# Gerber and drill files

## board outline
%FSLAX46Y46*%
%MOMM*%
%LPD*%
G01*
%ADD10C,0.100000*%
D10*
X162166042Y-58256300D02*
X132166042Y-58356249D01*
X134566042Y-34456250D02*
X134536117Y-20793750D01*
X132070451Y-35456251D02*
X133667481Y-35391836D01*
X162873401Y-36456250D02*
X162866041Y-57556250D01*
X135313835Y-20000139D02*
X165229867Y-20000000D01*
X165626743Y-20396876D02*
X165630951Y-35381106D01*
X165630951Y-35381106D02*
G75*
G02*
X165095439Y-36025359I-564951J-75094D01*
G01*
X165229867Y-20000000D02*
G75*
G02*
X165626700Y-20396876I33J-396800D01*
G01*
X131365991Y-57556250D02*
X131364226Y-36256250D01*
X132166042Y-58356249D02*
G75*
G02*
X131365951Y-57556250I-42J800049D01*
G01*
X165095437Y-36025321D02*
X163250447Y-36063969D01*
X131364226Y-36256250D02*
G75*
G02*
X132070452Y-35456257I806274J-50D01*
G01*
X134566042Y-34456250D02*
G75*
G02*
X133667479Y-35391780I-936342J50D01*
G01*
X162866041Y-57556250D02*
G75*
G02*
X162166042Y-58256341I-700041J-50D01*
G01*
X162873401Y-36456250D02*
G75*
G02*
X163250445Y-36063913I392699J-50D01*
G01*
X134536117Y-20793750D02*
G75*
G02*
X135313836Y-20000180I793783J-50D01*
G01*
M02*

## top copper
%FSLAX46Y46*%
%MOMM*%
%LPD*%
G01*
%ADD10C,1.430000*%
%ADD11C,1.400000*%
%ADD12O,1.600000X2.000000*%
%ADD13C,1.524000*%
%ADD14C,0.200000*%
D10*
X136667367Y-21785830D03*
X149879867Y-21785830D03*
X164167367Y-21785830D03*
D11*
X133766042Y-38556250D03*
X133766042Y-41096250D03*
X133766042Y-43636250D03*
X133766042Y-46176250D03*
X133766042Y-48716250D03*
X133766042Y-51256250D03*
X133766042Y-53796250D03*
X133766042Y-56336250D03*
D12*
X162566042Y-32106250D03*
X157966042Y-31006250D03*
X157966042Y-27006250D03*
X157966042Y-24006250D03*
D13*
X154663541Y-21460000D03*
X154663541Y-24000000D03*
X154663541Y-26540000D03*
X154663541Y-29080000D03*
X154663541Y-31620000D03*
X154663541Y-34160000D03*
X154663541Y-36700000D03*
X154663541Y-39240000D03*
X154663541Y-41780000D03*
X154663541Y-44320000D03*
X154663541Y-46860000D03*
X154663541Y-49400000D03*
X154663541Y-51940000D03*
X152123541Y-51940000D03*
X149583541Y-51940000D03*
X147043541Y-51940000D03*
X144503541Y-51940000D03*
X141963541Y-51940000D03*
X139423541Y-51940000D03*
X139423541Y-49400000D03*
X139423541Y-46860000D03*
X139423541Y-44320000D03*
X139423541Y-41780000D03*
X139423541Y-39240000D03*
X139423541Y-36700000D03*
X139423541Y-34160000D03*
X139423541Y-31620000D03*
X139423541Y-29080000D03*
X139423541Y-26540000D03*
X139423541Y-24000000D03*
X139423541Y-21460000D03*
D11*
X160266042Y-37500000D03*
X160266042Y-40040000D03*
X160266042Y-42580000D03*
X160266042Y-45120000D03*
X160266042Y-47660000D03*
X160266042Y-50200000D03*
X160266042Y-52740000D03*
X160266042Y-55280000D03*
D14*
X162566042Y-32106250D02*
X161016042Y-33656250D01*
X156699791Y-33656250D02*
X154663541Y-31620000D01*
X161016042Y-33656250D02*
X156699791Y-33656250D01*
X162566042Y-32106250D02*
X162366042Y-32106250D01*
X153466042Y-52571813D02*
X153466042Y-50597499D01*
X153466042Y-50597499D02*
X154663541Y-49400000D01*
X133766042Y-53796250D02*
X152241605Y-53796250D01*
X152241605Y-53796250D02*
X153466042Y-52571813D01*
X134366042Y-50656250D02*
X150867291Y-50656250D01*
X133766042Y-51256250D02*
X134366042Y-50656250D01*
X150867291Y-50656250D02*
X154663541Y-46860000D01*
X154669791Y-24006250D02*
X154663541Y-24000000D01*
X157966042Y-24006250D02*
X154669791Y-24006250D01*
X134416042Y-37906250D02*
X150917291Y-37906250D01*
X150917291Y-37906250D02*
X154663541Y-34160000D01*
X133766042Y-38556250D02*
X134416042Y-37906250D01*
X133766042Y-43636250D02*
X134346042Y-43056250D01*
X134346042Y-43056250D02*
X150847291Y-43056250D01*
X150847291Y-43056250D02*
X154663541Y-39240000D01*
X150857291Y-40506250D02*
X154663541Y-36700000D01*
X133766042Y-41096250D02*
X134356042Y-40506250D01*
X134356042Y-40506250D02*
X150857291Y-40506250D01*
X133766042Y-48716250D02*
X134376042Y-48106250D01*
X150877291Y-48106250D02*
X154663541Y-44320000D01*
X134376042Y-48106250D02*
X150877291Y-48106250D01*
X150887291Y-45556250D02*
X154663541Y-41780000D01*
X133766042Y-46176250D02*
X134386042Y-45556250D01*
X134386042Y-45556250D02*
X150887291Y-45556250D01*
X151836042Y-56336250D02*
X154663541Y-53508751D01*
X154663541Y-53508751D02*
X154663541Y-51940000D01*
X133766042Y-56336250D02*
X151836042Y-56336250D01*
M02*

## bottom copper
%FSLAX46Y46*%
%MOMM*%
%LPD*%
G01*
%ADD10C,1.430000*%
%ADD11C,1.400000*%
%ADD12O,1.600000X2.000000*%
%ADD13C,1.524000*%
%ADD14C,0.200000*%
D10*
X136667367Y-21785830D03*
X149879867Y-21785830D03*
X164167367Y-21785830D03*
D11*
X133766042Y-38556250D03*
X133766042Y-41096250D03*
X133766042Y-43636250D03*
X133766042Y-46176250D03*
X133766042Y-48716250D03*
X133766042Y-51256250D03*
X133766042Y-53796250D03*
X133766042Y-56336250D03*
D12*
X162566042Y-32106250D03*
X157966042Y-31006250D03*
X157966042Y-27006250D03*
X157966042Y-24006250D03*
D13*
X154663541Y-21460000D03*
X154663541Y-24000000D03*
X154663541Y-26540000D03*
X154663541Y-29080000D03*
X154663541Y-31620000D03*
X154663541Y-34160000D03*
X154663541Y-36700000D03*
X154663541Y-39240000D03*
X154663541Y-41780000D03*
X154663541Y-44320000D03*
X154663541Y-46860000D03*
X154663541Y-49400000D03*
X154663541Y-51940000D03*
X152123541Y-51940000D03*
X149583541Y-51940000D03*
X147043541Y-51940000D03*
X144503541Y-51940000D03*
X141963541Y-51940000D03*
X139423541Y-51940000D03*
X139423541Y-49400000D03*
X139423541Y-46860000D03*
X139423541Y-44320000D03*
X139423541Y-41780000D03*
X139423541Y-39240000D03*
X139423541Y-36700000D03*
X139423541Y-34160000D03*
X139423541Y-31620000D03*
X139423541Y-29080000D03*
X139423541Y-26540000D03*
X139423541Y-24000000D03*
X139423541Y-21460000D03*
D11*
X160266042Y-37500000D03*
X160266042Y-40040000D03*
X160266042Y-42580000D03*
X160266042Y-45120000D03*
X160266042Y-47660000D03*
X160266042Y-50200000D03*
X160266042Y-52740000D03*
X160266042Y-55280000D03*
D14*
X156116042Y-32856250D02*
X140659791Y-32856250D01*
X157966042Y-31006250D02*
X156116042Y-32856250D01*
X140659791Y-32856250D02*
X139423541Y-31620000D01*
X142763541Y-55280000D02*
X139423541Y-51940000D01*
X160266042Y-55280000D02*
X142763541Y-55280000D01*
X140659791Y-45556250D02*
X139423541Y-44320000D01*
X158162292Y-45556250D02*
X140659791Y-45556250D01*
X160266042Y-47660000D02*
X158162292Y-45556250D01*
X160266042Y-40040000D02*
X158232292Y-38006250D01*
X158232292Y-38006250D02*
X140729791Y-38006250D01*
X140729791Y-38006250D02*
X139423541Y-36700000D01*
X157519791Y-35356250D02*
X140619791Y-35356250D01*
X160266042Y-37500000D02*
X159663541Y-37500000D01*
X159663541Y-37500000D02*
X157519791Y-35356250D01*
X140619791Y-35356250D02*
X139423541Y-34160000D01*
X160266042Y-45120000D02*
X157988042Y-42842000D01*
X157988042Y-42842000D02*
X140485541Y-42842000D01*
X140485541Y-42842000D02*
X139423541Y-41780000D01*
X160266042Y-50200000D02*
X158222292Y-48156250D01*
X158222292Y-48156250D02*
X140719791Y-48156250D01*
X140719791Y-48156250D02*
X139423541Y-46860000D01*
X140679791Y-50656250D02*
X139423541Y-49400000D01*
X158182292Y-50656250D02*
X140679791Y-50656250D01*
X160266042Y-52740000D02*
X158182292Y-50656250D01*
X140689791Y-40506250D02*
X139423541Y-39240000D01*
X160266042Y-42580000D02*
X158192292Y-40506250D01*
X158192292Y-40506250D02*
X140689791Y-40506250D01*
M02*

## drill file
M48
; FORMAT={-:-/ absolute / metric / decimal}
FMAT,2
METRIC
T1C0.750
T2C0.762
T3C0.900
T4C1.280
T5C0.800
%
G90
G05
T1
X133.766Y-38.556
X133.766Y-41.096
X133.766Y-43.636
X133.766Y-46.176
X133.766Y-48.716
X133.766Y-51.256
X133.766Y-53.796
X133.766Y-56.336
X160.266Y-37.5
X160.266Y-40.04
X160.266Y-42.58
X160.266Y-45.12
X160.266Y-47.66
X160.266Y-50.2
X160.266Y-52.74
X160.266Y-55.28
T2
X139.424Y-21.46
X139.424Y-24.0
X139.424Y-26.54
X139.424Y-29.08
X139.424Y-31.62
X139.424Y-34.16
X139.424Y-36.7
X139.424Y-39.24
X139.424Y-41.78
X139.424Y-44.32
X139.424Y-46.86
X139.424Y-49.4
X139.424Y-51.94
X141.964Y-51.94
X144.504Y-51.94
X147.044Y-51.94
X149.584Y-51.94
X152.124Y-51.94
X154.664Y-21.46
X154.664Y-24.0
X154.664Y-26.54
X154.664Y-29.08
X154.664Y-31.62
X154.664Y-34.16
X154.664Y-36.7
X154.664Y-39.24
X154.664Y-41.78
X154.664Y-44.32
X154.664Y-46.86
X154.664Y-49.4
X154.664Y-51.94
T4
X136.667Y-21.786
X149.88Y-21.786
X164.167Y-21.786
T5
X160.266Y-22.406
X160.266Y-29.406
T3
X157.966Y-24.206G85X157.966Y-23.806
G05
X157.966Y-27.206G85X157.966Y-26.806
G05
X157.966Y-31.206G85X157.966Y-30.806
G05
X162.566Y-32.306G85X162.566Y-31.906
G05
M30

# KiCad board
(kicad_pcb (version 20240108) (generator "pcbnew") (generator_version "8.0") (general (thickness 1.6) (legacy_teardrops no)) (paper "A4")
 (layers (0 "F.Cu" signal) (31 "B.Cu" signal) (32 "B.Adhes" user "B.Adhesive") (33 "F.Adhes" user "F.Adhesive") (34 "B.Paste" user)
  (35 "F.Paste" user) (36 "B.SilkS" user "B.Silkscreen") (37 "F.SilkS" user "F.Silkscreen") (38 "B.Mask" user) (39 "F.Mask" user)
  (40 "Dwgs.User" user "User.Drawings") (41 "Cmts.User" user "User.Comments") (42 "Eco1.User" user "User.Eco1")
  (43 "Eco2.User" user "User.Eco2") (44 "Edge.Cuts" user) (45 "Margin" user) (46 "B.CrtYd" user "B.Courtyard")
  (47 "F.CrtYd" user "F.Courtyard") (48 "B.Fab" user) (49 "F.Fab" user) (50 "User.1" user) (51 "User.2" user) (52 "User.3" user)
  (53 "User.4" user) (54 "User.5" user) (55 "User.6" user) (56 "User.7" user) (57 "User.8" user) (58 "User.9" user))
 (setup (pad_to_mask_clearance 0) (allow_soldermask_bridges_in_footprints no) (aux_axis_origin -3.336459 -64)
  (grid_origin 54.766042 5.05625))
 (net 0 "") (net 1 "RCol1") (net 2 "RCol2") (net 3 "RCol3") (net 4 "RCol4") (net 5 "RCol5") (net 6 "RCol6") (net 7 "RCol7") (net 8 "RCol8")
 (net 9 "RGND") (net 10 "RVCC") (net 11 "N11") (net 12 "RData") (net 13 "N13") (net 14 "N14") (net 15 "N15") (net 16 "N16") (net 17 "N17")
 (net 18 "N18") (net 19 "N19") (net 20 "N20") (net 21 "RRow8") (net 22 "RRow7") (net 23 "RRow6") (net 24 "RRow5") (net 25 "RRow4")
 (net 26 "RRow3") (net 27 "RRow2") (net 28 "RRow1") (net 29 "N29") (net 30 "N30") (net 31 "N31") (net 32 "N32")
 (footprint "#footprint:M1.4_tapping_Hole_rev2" (layer "F.Cu") (at 146.916042 21.90625 -90)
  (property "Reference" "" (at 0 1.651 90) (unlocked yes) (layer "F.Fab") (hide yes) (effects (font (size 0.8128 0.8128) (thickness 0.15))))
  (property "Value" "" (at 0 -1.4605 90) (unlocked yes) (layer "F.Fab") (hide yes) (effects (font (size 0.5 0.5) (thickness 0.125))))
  (pad "" thru_hole circle (at -0.12042 10.248675 270) (size 1.43 1.43) (drill 1.28) (layers "*.Cu" "*.Mask") (remove_unused_layers no)))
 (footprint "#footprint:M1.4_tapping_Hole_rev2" (layer "F.Cu") (at 149.879867 21.78583 -90)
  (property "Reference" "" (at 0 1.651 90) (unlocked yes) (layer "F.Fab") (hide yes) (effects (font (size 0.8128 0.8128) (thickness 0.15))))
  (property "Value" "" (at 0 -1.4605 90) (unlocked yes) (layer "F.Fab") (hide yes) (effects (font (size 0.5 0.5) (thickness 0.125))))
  (pad "" thru_hole circle (at 0 0 270) (size 1.43 1.43) (drill 1.28) (layers "*.Cu" "*.Mask") (remove_unused_layers no)))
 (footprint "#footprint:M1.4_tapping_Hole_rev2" (layer "F.Cu") (at 164.167367 21.78583 -90)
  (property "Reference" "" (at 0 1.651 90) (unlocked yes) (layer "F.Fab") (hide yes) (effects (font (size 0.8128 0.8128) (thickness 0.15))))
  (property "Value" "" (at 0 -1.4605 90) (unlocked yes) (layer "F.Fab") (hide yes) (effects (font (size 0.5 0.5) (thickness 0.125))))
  (pad "" thru_hole circle (at 0 0 270) (size 1.43 1.43) (drill 1.28) (layers "*.Cu" "*.Mask") (remove_unused_layers no)))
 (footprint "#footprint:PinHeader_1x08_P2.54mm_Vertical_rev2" (layer "B.Cu") (at 133.766042 38.55625 180)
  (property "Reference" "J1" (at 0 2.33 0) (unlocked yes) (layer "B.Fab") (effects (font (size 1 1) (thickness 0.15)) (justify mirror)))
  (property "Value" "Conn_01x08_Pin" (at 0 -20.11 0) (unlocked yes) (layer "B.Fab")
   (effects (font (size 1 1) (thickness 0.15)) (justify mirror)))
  (pad "1" thru_hole circle (at 0 0 180) (size 1.4 1.4) (drill 0.75) (layers "*.Cu" "*.Mask") (remove_unused_layers no) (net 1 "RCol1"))
  (pad "2" thru_hole circle (at 0 -2.54 180) (size 1.4 1.4) (drill 0.75) (layers "*.Cu" "*.Mask") (remove_unused_layers no) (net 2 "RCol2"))
  (pad "3" thru_hole circle (at 0 -5.08 180) (size 1.4 1.4) (drill 0.75) (layers "*.Cu" "*.Mask") (remove_unused_layers no) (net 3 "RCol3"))
  (pad "4" thru_hole circle (at 0 -7.62 180) (size 1.4 1.4) (drill 0.75) (layers "*.Cu" "*.Mask") (remove_unused_layers no) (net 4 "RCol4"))
  (pad "5" thru_hole circle (at 0 -10.16 180) (size 1.4 1.4) (drill 0.75) (layers "*.Cu" "*.Mask") (remove_unused_layers no) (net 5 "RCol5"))
  (pad "6" thru_hole circle (at 0 -12.7 180) (size 1.4 1.4) (drill 0.75) (layers "*.Cu" "*.Mask") (remove_unused_layers no) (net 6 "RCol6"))
  (pad "7" thru_hole circle (at 0 -15.24 180) (size 1.4 1.4) (drill 0.75) (layers "*.Cu" "*.Mask") (remove_unused_layers no) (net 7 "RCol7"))
  (pad "8" thru_hole circle (at 0 -17.78 180) (size 1.4 1.4) (drill 0.75) (layers "*.Cu" "*.Mask") (remove_unused_layers no) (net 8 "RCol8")))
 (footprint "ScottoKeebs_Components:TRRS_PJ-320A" (layer "B.Cu") (at 160.266042 20.80625 180)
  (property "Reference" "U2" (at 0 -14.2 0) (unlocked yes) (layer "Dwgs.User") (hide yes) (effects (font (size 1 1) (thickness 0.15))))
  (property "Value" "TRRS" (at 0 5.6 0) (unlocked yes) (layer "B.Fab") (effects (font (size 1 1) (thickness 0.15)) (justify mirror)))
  (pad "" np_thru_hole circle (at 0 -8.6 180) (size 0.8 0.8) (drill 0.8) (layers "*.Cu" "*.Mask"))
  (pad "" np_thru_hole circle (at 0 -1.6 180) (size 0.8 0.8) (drill 0.8) (layers "*.Cu" "*.Mask"))
  (pad "1" thru_hole oval (at -2.3 -11.3 180) (size 1.6 2) (drill oval 0.9 1.3) (layers "*.Cu" "*.Mask") (remove_unused_layers no)
   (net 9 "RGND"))
  (pad "2" thru_hole oval (at 2.3 -10.2 180) (size 1.6 2) (drill oval 0.9 1.3) (layers "*.Cu" "*.Mask") (remove_unused_layers no)
   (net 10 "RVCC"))
  (pad "3" thru_hole oval (at 2.3 -6.2 180) (size 1.6 2) (drill oval 0.9 1.3) (layers "*.Cu" "*.Mask") (remove_unused_layers no)
   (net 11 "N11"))
  (pad "4" thru_hole oval (at 2.3 -3.2 180) (size 1.6 2) (drill oval 0.9 1.3) (layers "*.Cu" "*.Mask") (remove_unused_layers no)
   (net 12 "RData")))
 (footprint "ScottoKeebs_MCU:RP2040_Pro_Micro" (layer "B.Cu") (at 147.043541 37.97 180)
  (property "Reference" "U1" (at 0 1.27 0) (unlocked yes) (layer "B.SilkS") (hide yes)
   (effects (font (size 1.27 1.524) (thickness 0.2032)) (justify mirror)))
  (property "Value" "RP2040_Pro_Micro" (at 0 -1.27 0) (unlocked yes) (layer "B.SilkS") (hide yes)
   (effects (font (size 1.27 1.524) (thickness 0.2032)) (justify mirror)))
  (pad "1" thru_hole circle (at -7.62 16.51 180) (size 1.524 1.524) (drill 0.762) (layers "*.Cu" "*.Mask") (remove_unused_layers no)
   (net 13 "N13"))
  (pad "2" thru_hole circle (at -7.62 13.97 180) (size 1.524 1.524) (drill 0.762) (layers "*.Cu" "*.Mask") (remove_unused_layers no)
   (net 12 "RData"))
  (pad "3" thru_hole circle (at -7.62 11.43 180) (size 1.524 1.524) (drill 0.762) (layers "*.Cu" "*.Mask") (remove_unused_layers no)
   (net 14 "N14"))
  (pad "4" thru_hole circle (at -7.62 8.89 180) (size 1.524 1.524) (drill 0.762) (layers "*.Cu" "*.Mask") (remove_unused_layers no)
   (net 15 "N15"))
  (pad "5" thru_hole circle (at -7.62 6.35 180) (size 1.524 1.524) (drill 0.762) (layers "*.Cu" "*.Mask") (remove_unused_layers no)
   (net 9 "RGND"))
  (pad "6" thru_hole circle (at -7.62 3.81 180) (size 1.524 1.524) (drill 0.762) (layers "*.Cu" "*.Mask") (remove_unused_layers no)
   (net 1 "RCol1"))
  (pad "7" thru_hole circle (at -7.62 1.27 180) (size 1.524 1.524) (drill 0.762) (layers "*.Cu" "*.Mask") (remove_unused_layers no)
   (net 2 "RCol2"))
  (pad "8" thru_hole circle (at -7.62 -1.27 180) (size 1.524 1.524) (drill 0.762) (layers "*.Cu" "*.Mask") (remove_unused_layers no)
   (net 3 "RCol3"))
  (pad "9" thru_hole circle (at -7.62 -3.81 180) (size 1.524 1.524) (drill 0.762) (layers "*.Cu" "*.Mask") (remove_unused_layers no)
   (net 4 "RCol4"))
  (pad "10" thru_hole circle (at -7.62 -6.35 180) (size 1.524 1.524) (drill 0.762) (layers "*.Cu" "*.Mask") (remove_unused_layers no)
   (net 5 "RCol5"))
  (pad "11" thru_hole circle (at -7.62 -8.89 180) (size 1.524 1.524) (drill 0.762) (layers "*.Cu" "*.Mask") (remove_unused_layers no)
   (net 6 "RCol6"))
  (pad "12" thru_hole circle (at -7.62 -11.43 180) (size 1.524 1.524) (drill 0.762) (layers "*.Cu" "*.Mask") (remove_unused_layers no)
   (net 7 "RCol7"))
  (pad "13" thru_hole circle (at -7.62 -13.97 180) (size 1.524 1.524) (drill 0.762) (layers "*.Cu" "*.Mask") (remove_unused_layers no)
   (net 8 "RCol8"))
  (pad "14" thru_hole circle (at -5.08 -13.97 180) (size 1.524 1.524) (drill 0.762) (layers "*.Cu" "*.Mask") (remove_unused_layers no)
   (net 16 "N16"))
  (pad "15" thru_hole circle (at -2.54 -13.97 180) (size 1.524 1.524) (drill 0.762) (layers "*.Cu" "*.Mask") (remove_unused_layers no)
   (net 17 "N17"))
  (pad "16" thru_hole circle (at 0 -13.97 180) (size 1.524 1.524) (drill 0.762) (layers "*.Cu" "*.Mask") (remove_unused_layers no)
   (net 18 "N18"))
  (pad "17" thru_hole circle (at 2.54 -13.97 180) (size 1.524 1.524) (drill 0.762) (layers "*.Cu" "*.Mask") (remove_unused_layers no)
   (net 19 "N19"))
  (pad "18" thru_hole circle (at 5.08 -13.97 180) (size 1.524 1.524) (drill 0.762) (layers "*.Cu" "*.Mask") (remove_unused_layers no)
   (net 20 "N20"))
  (pad "19" thru_hole circle (at 7.62 -13.97 180) (size 1.524 1.524) (drill 0.762) (layers "*.Cu" "*.Mask") (remove_unused_layers no)
   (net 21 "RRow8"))
  (pad "20" thru_hole circle (at 7.62 -11.43 180) (size 1.524 1.524) (drill 0.762) (layers "*.Cu" "*.Mask") (remove_unused_layers no)
   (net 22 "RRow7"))
  (pad "21" thru_hole circle (at 7.62 -8.89 180) (size 1.524 1.524) (drill 0.762) (layers "*.Cu" "*.Mask") (remove_unused_layers no)
   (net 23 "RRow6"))
  (pad "22" thru_hole circle (at 7.62 -6.35 180) (size 1.524 1.524) (drill 0.762) (layers "*.Cu" "*.Mask") (remove_unused_layers no)
   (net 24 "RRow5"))
  (pad "23" thru_hole circle (at 7.62 -3.81 180) (size 1.524 1.524) (drill 0.762) (layers "*.Cu" "*.Mask") (remove_unused_layers no)
   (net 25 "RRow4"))
  (pad "24" thru_hole circle (at 7.62 -1.27 180) (size 1.524 1.524) (drill 0.762) (layers "*.Cu" "*.Mask") (remove_unused_layers no)
   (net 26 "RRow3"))
  (pad "25" thru_hole circle (at 7.62 1.27 180) (size 1.524 1.524) (drill 0.762) (layers "*.Cu" "*.Mask") (remove_unused_layers no)
   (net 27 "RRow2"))
  (pad "26" thru_hole circle (at 7.62 3.81 180) (size 1.524 1.524) (drill 0.762) (layers "*.Cu" "*.Mask") (remove_unused_layers no)
   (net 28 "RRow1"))
  (pad "27" thru_hole circle (at 7.62 6.35 180) (size 1.524 1.524) (drill 0.762) (layers "*.Cu" "*.Mask") (remove_unused_layers no)
   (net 10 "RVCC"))
  (pad "28" thru_hole circle (at 7.62 8.89 180) (size 1.524 1.524) (drill 0.762) (layers "*.Cu" "*.Mask") (remove_unused_layers no)
   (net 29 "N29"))
  (pad "29" thru_hole circle (at 7.62 11.43 180) (size 1.524 1.524) (drill 0.762) (layers "*.Cu" "*.Mask") (remove_unused_layers no)
   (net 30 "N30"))
  (pad "30" thru_hole circle (at 7.62 13.97 180) (size 1.524 1.524) (drill 0.762) (layers "*.Cu" "*.Mask") (remove_unused_layers no)
   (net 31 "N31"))
  (pad "31" thru_hole circle (at 7.62 16.51 180) (size 1.524 1.524) (drill 0.762) (layers "*.Cu" "*.Mask") (remove_unused_layers no)
   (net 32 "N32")))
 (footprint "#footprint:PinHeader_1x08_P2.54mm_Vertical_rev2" (layer "B.Cu") (at 160.266042 37.5 180)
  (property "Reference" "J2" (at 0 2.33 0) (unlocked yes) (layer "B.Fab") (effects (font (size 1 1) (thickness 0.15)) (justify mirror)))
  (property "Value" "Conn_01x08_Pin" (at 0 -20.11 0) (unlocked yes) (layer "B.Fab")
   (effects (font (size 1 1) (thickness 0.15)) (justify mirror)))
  (pad "1" thru_hole circle (at 0 0 180) (size 1.4 1.4) (drill 0.75) (layers "*.Cu" "*.Mask") (remove_unused_layers no) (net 28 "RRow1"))
  (pad "2" thru_hole circle (at 0 -2.54 180) (size 1.4 1.4) (drill 0.75) (layers "*.Cu" "*.Mask") (remove_unused_layers no) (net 27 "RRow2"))
  (pad "3" thru_hole circle (at 0 -5.08 180) (size 1.4 1.4) (drill 0.75) (layers "*.Cu" "*.Mask") (remove_unused_layers no) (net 26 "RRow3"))
  (pad "4" thru_hole circle (at 0 -7.62 180) (size 1.4 1.4) (drill 0.75) (layers "*.Cu" "*.Mask") (remove_unused_layers no) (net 25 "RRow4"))
  (pad "5" thru_hole circle (at 0 -10.16 180) (size 1.4 1.4) (drill 0.75) (layers "*.Cu" "*.Mask") (remove_unused_layers no)
   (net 24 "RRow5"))
  (pad "6" thru_hole circle (at 0 -12.7 180) (size 1.4 1.4) (drill 0.75) (layers "*.Cu" "*.Mask") (remove_unused_layers no) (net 23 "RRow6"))
  (pad "7" thru_hole circle (at 0 -15.24 180) (size 1.4 1.4) (drill 0.75) (layers "*.Cu" "*.Mask") (remove_unused_layers no)
   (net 22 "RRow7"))
  (pad "8" thru_hole circle (at 0 -17.78 180) (size 1.4 1.4) (drill 0.75) (layers "*.Cu" "*.Mask") (remove_unused_layers no)
   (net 21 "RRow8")))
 (gr_line (start 162.166042 58.2563) (end 132.166042 58.356249) (stroke (width 0.1) (type default)) (layer "Edge.Cuts"))
 (gr_line (start 134.566042 34.45625) (end 134.536117 20.79375) (stroke (width 0.1) (type default)) (layer "Edge.Cuts"))
 (gr_line (start 132.070451 35.456251) (end 133.667481 35.391836) (stroke (width 0.1) (type default)) (layer "Edge.Cuts"))
 (gr_line (start 162.873401 36.45625) (end 162.866041 57.55625) (stroke (width 0.1) (type default)) (layer "Edge.Cuts"))
 (gr_line (start 135.313835 20.000139) (end 165.229867 20) (stroke (width 0.1) (type default)) (layer "Edge.Cuts"))
 (gr_line (start 165.626743 20.396876) (end 165.630951 35.381106) (stroke (width 0.1) (type default)) (layer "Edge.Cuts"))
 (gr_arc (start 165.630951 35.381106) (mid 165.50428 35.820493) (end 165.095437 36.025321) (stroke (width 0.1) (type default))
  (layer "Edge.Cuts"))
 (gr_arc (start 165.229867 20) (mid 165.510522 20.11622) (end 165.626743 20.396876) (stroke (width 0.1) (type default)) (layer "Edge.Cuts"))
 (gr_line (start 131.365991 57.55625) (end 131.364226 36.25625) (stroke (width 0.1) (type default)) (layer "Edge.Cuts"))
 (gr_arc (start 132.166042 58.356249) (mid 131.600338 58.121938) (end 131.365991 57.55625) (stroke (width 0.1) (type default))
  (layer "Edge.Cuts"))
 (gr_line (start 165.095437 36.025321) (end 163.250447 36.063969) (stroke (width 0.1) (type default)) (layer "Edge.Cuts"))
 (gr_arc (start 131.364226 36.25625) (mid 131.566051 35.722696) (end 132.070451 35.456251) (stroke (width 0.1) (type default))
  (layer "Edge.Cuts"))
 (gr_arc (start 134.566042 34.45625) (mid 134.305008 35.104851) (end 133.667481 35.391836) (stroke (width 0.1) (type default))
  (layer "Edge.Cuts"))
 (gr_arc (start 162.866041 57.55625) (mid 162.661034 58.051257) (end 162.166042 58.2563) (stroke (width 0.1) (type default))
  (layer "Edge.Cuts"))
 (gr_arc (start 162.873401 36.45625) (mid 162.982963 36.184226) (end 163.250447 36.063969) (stroke (width 0.1) (type default))
  (layer "Edge.Cuts"))
 (gr_arc (start 134.536117 20.79375) (mid 134.762974 20.238187) (end 135.313835 20.000139) (stroke (width 0.1) (type default))
  (layer "Edge.Cuts"))
 (segment (start 162.566042 32.10625) (end 161.016042 33.65625) (width 0.2) (layer "F.Cu") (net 9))
 (segment (start 156.699791 33.65625) (end 154.663541 31.62) (width 0.2) (layer "F.Cu") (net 9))
 (segment (start 161.016042 33.65625) (end 156.699791 33.65625) (width 0.2) (layer "F.Cu") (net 9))
 (segment (start 162.566042 32.10625) (end 162.366042 32.10625) (width 0.2) (layer "F.Cu") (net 9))
 (segment (start 156.116042 32.85625) (end 140.659791 32.85625) (width 0.2) (layer "B.Cu") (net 10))
 (segment (start 157.966042 31.00625) (end 156.116042 32.85625) (width 0.2) (layer "B.Cu") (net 10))
 (segment (start 140.659791 32.85625) (end 139.423541 31.62) (width 0.2) (layer "B.Cu") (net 10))
 (segment (start 142.763541 55.28) (end 139.423541 51.94) (width 0.2) (layer "B.Cu") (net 21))
 (segment (start 160.266042 55.28) (end 142.763541 55.28) (width 0.2) (layer "B.Cu") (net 21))
 (segment (start 140.659791 45.55625) (end 139.423541 44.32) (width 0.2) (layer "B.Cu") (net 24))
 (segment (start 158.162292 45.55625) (end 140.659791 45.55625) (width 0.2) (layer "B.Cu") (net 24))
 (segment (start 160.266042 47.66) (end 158.162292 45.55625) (width 0.2) (layer "B.Cu") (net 24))
 (segment (start 153.466042 52.571813) (end 153.466042 50.597499) (width 0.2) (layer "F.Cu") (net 7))
 (segment (start 153.466042 50.597499) (end 154.663541 49.4) (width 0.2) (layer "F.Cu") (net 7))
 (segment (start 133.766042 53.79625) (end 152.241605 53.79625) (width 0.2) (layer "F.Cu") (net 7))
 (segment (start 152.241605 53.79625) (end 153.466042 52.571813) (width 0.2) (layer "F.Cu") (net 7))
 (segment (start 134.366042 50.65625) (end 150.867291 50.65625) (width 0.2) (layer "F.Cu") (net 6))
 (segment (start 133.766042 51.25625) (end 134.366042 50.65625) (width 0.2) (layer "F.Cu") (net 6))
 (segment (start 150.867291 50.65625) (end 154.663541 46.86) (width 0.2) (layer "F.Cu") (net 6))
 (segment (start 160.266042 40.04) (end 158.232292 38.00625) (width 0.2) (layer "B.Cu") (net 27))
 (segment (start 158.232292 38.00625) (end 140.729791 38.00625) (width 0.2) (layer "B.Cu") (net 27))
 (segment (start 140.729791 38.00625) (end 139.423541 36.7) (width 0.2) (layer "B.Cu") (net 27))
 (segment (start 154.669791 24.00625) (end 154.663541 24) (width 0.2) (layer "F.Cu") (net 12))
 (segment (start 157.966042 24.00625) (end 154.669791 24.00625) (width 0.2) (layer "F.Cu") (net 12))
 (segment (start 134.416042 37.90625) (end 150.917291 37.90625) (width 0.2) (layer "F.Cu") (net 1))
 (segment (start 150.917291 37.90625) (end 154.663541 34.16) (width 0.2) (layer "F.Cu") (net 1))
 (segment (start 133.766042 38.55625) (end 134.416042 37.90625) (width 0.2) (layer "F.Cu") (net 1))
 (segment (start 157.519791 35.35625) (end 140.619791 35.35625) (width 0.2) (layer "B.Cu") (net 28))
 (segment (start 160.266042 37.5) (end 159.663541 37.5) (width 0.2) (layer "B.Cu") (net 28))
 (segment (start 159.663541 37.5) (end 157.519791 35.35625) (width 0.2) (layer "B.Cu") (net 28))
 (segment (start 140.619791 35.35625) (end 139.423541 34.16) (width 0.2) (layer "B.Cu") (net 28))
 (segment (start 133.766042 43.63625) (end 134.346042 43.05625) (width 0.2) (layer "F.Cu") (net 3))
 (segment (start 134.346042 43.05625) (end 150.847291 43.05625) (width 0.2) (layer "F.Cu") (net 3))
 (segment (start 150.847291 43.05625) (end 154.663541 39.24) (width 0.2) (layer "F.Cu") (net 3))
 (segment (start 160.266042 45.12) (end 157.988042 42.842) (width 0.2) (layer "B.Cu") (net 25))
 (segment (start 157.988042 42.842) (end 140.485541 42.842) (width 0.2) (layer "B.Cu") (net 25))
 (segment (start 140.485541 42.842) (end 139.423541 41.78) (width 0.2) (layer "B.Cu") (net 25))
 (segment (start 160.266042 50.2) (end 158.222292 48.15625) (width 0.2) (layer "B.Cu") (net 23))
 (segment (start 158.222292 48.15625) (end 140.719791 48.15625) (width 0.2) (layer "B.Cu") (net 23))
 (segment (start 140.719791 48.15625) (end 139.423541 46.86) (width 0.2) (layer "B.Cu") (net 23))
 (segment (start 150.857291 40.50625) (end 154.663541 36.7) (width 0.2) (layer "F.Cu") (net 2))
 (segment (start 133.766042 41.09625) (end 134.356042 40.50625) (width 0.2) (layer "F.Cu") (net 2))
 (segment (start 134.356042 40.50625) (end 150.857291 40.50625) (width 0.2) (layer "F.Cu") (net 2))
 (segment (start 133.766042 48.71625) (end 134.376042 48.10625) (width 0.2) (layer "F.Cu") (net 5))
 (segment (start 150.877291 48.10625) (end 154.663541 44.32) (width 0.2) (layer "F.Cu") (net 5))
 (segment (start 134.376042 48.10625) (end 150.877291 48.10625) (width 0.2) (layer "F.Cu") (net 5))
 (segment (start 150.887291 45.55625) (end 154.663541 41.78) (width 0.2) (layer "F.Cu") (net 4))
 (segment (start 133.766042 46.17625) (end 134.386042 45.55625) (width 0.2) (layer "F.Cu") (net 4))
 (segment (start 134.386042 45.55625) (end 150.887291 45.55625) (width 0.2) (layer "F.Cu") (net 4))
 (segment (start 140.679791 50.65625) (end 139.423541 49.4) (width 0.2) (layer "B.Cu") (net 22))
 (segment (start 158.182292 50.65625) (end 140.679791 50.65625) (width 0.2) (layer "B.Cu") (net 22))
 (segment (start 160.266042 52.74) (end 158.182292 50.65625) (width 0.2) (layer "B.Cu") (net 22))
 (segment (start 140.689791 40.50625) (end 139.423541 39.24) (width 0.2) (layer "B.Cu") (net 26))
 (segment (start 160.266042 42.58) (end 158.192292 40.50625) (width 0.2) (layer "B.Cu") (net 26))
 (segment (start 158.192292 40.50625) (end 140.689791 40.50625) (width 0.2) (layer "B.Cu") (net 26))
 (segment (start 151.836042 56.33625) (end 154.663541 53.508751) (width 0.2) (layer "F.Cu") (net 8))
 (segment (start 154.663541 53.508751) (end 154.663541 51.94) (width 0.2) (layer "F.Cu") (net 8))
 (segment (start 133.766042 56.33625) (end 151.836042 56.33625) (width 0.2) (layer "F.Cu") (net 8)))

